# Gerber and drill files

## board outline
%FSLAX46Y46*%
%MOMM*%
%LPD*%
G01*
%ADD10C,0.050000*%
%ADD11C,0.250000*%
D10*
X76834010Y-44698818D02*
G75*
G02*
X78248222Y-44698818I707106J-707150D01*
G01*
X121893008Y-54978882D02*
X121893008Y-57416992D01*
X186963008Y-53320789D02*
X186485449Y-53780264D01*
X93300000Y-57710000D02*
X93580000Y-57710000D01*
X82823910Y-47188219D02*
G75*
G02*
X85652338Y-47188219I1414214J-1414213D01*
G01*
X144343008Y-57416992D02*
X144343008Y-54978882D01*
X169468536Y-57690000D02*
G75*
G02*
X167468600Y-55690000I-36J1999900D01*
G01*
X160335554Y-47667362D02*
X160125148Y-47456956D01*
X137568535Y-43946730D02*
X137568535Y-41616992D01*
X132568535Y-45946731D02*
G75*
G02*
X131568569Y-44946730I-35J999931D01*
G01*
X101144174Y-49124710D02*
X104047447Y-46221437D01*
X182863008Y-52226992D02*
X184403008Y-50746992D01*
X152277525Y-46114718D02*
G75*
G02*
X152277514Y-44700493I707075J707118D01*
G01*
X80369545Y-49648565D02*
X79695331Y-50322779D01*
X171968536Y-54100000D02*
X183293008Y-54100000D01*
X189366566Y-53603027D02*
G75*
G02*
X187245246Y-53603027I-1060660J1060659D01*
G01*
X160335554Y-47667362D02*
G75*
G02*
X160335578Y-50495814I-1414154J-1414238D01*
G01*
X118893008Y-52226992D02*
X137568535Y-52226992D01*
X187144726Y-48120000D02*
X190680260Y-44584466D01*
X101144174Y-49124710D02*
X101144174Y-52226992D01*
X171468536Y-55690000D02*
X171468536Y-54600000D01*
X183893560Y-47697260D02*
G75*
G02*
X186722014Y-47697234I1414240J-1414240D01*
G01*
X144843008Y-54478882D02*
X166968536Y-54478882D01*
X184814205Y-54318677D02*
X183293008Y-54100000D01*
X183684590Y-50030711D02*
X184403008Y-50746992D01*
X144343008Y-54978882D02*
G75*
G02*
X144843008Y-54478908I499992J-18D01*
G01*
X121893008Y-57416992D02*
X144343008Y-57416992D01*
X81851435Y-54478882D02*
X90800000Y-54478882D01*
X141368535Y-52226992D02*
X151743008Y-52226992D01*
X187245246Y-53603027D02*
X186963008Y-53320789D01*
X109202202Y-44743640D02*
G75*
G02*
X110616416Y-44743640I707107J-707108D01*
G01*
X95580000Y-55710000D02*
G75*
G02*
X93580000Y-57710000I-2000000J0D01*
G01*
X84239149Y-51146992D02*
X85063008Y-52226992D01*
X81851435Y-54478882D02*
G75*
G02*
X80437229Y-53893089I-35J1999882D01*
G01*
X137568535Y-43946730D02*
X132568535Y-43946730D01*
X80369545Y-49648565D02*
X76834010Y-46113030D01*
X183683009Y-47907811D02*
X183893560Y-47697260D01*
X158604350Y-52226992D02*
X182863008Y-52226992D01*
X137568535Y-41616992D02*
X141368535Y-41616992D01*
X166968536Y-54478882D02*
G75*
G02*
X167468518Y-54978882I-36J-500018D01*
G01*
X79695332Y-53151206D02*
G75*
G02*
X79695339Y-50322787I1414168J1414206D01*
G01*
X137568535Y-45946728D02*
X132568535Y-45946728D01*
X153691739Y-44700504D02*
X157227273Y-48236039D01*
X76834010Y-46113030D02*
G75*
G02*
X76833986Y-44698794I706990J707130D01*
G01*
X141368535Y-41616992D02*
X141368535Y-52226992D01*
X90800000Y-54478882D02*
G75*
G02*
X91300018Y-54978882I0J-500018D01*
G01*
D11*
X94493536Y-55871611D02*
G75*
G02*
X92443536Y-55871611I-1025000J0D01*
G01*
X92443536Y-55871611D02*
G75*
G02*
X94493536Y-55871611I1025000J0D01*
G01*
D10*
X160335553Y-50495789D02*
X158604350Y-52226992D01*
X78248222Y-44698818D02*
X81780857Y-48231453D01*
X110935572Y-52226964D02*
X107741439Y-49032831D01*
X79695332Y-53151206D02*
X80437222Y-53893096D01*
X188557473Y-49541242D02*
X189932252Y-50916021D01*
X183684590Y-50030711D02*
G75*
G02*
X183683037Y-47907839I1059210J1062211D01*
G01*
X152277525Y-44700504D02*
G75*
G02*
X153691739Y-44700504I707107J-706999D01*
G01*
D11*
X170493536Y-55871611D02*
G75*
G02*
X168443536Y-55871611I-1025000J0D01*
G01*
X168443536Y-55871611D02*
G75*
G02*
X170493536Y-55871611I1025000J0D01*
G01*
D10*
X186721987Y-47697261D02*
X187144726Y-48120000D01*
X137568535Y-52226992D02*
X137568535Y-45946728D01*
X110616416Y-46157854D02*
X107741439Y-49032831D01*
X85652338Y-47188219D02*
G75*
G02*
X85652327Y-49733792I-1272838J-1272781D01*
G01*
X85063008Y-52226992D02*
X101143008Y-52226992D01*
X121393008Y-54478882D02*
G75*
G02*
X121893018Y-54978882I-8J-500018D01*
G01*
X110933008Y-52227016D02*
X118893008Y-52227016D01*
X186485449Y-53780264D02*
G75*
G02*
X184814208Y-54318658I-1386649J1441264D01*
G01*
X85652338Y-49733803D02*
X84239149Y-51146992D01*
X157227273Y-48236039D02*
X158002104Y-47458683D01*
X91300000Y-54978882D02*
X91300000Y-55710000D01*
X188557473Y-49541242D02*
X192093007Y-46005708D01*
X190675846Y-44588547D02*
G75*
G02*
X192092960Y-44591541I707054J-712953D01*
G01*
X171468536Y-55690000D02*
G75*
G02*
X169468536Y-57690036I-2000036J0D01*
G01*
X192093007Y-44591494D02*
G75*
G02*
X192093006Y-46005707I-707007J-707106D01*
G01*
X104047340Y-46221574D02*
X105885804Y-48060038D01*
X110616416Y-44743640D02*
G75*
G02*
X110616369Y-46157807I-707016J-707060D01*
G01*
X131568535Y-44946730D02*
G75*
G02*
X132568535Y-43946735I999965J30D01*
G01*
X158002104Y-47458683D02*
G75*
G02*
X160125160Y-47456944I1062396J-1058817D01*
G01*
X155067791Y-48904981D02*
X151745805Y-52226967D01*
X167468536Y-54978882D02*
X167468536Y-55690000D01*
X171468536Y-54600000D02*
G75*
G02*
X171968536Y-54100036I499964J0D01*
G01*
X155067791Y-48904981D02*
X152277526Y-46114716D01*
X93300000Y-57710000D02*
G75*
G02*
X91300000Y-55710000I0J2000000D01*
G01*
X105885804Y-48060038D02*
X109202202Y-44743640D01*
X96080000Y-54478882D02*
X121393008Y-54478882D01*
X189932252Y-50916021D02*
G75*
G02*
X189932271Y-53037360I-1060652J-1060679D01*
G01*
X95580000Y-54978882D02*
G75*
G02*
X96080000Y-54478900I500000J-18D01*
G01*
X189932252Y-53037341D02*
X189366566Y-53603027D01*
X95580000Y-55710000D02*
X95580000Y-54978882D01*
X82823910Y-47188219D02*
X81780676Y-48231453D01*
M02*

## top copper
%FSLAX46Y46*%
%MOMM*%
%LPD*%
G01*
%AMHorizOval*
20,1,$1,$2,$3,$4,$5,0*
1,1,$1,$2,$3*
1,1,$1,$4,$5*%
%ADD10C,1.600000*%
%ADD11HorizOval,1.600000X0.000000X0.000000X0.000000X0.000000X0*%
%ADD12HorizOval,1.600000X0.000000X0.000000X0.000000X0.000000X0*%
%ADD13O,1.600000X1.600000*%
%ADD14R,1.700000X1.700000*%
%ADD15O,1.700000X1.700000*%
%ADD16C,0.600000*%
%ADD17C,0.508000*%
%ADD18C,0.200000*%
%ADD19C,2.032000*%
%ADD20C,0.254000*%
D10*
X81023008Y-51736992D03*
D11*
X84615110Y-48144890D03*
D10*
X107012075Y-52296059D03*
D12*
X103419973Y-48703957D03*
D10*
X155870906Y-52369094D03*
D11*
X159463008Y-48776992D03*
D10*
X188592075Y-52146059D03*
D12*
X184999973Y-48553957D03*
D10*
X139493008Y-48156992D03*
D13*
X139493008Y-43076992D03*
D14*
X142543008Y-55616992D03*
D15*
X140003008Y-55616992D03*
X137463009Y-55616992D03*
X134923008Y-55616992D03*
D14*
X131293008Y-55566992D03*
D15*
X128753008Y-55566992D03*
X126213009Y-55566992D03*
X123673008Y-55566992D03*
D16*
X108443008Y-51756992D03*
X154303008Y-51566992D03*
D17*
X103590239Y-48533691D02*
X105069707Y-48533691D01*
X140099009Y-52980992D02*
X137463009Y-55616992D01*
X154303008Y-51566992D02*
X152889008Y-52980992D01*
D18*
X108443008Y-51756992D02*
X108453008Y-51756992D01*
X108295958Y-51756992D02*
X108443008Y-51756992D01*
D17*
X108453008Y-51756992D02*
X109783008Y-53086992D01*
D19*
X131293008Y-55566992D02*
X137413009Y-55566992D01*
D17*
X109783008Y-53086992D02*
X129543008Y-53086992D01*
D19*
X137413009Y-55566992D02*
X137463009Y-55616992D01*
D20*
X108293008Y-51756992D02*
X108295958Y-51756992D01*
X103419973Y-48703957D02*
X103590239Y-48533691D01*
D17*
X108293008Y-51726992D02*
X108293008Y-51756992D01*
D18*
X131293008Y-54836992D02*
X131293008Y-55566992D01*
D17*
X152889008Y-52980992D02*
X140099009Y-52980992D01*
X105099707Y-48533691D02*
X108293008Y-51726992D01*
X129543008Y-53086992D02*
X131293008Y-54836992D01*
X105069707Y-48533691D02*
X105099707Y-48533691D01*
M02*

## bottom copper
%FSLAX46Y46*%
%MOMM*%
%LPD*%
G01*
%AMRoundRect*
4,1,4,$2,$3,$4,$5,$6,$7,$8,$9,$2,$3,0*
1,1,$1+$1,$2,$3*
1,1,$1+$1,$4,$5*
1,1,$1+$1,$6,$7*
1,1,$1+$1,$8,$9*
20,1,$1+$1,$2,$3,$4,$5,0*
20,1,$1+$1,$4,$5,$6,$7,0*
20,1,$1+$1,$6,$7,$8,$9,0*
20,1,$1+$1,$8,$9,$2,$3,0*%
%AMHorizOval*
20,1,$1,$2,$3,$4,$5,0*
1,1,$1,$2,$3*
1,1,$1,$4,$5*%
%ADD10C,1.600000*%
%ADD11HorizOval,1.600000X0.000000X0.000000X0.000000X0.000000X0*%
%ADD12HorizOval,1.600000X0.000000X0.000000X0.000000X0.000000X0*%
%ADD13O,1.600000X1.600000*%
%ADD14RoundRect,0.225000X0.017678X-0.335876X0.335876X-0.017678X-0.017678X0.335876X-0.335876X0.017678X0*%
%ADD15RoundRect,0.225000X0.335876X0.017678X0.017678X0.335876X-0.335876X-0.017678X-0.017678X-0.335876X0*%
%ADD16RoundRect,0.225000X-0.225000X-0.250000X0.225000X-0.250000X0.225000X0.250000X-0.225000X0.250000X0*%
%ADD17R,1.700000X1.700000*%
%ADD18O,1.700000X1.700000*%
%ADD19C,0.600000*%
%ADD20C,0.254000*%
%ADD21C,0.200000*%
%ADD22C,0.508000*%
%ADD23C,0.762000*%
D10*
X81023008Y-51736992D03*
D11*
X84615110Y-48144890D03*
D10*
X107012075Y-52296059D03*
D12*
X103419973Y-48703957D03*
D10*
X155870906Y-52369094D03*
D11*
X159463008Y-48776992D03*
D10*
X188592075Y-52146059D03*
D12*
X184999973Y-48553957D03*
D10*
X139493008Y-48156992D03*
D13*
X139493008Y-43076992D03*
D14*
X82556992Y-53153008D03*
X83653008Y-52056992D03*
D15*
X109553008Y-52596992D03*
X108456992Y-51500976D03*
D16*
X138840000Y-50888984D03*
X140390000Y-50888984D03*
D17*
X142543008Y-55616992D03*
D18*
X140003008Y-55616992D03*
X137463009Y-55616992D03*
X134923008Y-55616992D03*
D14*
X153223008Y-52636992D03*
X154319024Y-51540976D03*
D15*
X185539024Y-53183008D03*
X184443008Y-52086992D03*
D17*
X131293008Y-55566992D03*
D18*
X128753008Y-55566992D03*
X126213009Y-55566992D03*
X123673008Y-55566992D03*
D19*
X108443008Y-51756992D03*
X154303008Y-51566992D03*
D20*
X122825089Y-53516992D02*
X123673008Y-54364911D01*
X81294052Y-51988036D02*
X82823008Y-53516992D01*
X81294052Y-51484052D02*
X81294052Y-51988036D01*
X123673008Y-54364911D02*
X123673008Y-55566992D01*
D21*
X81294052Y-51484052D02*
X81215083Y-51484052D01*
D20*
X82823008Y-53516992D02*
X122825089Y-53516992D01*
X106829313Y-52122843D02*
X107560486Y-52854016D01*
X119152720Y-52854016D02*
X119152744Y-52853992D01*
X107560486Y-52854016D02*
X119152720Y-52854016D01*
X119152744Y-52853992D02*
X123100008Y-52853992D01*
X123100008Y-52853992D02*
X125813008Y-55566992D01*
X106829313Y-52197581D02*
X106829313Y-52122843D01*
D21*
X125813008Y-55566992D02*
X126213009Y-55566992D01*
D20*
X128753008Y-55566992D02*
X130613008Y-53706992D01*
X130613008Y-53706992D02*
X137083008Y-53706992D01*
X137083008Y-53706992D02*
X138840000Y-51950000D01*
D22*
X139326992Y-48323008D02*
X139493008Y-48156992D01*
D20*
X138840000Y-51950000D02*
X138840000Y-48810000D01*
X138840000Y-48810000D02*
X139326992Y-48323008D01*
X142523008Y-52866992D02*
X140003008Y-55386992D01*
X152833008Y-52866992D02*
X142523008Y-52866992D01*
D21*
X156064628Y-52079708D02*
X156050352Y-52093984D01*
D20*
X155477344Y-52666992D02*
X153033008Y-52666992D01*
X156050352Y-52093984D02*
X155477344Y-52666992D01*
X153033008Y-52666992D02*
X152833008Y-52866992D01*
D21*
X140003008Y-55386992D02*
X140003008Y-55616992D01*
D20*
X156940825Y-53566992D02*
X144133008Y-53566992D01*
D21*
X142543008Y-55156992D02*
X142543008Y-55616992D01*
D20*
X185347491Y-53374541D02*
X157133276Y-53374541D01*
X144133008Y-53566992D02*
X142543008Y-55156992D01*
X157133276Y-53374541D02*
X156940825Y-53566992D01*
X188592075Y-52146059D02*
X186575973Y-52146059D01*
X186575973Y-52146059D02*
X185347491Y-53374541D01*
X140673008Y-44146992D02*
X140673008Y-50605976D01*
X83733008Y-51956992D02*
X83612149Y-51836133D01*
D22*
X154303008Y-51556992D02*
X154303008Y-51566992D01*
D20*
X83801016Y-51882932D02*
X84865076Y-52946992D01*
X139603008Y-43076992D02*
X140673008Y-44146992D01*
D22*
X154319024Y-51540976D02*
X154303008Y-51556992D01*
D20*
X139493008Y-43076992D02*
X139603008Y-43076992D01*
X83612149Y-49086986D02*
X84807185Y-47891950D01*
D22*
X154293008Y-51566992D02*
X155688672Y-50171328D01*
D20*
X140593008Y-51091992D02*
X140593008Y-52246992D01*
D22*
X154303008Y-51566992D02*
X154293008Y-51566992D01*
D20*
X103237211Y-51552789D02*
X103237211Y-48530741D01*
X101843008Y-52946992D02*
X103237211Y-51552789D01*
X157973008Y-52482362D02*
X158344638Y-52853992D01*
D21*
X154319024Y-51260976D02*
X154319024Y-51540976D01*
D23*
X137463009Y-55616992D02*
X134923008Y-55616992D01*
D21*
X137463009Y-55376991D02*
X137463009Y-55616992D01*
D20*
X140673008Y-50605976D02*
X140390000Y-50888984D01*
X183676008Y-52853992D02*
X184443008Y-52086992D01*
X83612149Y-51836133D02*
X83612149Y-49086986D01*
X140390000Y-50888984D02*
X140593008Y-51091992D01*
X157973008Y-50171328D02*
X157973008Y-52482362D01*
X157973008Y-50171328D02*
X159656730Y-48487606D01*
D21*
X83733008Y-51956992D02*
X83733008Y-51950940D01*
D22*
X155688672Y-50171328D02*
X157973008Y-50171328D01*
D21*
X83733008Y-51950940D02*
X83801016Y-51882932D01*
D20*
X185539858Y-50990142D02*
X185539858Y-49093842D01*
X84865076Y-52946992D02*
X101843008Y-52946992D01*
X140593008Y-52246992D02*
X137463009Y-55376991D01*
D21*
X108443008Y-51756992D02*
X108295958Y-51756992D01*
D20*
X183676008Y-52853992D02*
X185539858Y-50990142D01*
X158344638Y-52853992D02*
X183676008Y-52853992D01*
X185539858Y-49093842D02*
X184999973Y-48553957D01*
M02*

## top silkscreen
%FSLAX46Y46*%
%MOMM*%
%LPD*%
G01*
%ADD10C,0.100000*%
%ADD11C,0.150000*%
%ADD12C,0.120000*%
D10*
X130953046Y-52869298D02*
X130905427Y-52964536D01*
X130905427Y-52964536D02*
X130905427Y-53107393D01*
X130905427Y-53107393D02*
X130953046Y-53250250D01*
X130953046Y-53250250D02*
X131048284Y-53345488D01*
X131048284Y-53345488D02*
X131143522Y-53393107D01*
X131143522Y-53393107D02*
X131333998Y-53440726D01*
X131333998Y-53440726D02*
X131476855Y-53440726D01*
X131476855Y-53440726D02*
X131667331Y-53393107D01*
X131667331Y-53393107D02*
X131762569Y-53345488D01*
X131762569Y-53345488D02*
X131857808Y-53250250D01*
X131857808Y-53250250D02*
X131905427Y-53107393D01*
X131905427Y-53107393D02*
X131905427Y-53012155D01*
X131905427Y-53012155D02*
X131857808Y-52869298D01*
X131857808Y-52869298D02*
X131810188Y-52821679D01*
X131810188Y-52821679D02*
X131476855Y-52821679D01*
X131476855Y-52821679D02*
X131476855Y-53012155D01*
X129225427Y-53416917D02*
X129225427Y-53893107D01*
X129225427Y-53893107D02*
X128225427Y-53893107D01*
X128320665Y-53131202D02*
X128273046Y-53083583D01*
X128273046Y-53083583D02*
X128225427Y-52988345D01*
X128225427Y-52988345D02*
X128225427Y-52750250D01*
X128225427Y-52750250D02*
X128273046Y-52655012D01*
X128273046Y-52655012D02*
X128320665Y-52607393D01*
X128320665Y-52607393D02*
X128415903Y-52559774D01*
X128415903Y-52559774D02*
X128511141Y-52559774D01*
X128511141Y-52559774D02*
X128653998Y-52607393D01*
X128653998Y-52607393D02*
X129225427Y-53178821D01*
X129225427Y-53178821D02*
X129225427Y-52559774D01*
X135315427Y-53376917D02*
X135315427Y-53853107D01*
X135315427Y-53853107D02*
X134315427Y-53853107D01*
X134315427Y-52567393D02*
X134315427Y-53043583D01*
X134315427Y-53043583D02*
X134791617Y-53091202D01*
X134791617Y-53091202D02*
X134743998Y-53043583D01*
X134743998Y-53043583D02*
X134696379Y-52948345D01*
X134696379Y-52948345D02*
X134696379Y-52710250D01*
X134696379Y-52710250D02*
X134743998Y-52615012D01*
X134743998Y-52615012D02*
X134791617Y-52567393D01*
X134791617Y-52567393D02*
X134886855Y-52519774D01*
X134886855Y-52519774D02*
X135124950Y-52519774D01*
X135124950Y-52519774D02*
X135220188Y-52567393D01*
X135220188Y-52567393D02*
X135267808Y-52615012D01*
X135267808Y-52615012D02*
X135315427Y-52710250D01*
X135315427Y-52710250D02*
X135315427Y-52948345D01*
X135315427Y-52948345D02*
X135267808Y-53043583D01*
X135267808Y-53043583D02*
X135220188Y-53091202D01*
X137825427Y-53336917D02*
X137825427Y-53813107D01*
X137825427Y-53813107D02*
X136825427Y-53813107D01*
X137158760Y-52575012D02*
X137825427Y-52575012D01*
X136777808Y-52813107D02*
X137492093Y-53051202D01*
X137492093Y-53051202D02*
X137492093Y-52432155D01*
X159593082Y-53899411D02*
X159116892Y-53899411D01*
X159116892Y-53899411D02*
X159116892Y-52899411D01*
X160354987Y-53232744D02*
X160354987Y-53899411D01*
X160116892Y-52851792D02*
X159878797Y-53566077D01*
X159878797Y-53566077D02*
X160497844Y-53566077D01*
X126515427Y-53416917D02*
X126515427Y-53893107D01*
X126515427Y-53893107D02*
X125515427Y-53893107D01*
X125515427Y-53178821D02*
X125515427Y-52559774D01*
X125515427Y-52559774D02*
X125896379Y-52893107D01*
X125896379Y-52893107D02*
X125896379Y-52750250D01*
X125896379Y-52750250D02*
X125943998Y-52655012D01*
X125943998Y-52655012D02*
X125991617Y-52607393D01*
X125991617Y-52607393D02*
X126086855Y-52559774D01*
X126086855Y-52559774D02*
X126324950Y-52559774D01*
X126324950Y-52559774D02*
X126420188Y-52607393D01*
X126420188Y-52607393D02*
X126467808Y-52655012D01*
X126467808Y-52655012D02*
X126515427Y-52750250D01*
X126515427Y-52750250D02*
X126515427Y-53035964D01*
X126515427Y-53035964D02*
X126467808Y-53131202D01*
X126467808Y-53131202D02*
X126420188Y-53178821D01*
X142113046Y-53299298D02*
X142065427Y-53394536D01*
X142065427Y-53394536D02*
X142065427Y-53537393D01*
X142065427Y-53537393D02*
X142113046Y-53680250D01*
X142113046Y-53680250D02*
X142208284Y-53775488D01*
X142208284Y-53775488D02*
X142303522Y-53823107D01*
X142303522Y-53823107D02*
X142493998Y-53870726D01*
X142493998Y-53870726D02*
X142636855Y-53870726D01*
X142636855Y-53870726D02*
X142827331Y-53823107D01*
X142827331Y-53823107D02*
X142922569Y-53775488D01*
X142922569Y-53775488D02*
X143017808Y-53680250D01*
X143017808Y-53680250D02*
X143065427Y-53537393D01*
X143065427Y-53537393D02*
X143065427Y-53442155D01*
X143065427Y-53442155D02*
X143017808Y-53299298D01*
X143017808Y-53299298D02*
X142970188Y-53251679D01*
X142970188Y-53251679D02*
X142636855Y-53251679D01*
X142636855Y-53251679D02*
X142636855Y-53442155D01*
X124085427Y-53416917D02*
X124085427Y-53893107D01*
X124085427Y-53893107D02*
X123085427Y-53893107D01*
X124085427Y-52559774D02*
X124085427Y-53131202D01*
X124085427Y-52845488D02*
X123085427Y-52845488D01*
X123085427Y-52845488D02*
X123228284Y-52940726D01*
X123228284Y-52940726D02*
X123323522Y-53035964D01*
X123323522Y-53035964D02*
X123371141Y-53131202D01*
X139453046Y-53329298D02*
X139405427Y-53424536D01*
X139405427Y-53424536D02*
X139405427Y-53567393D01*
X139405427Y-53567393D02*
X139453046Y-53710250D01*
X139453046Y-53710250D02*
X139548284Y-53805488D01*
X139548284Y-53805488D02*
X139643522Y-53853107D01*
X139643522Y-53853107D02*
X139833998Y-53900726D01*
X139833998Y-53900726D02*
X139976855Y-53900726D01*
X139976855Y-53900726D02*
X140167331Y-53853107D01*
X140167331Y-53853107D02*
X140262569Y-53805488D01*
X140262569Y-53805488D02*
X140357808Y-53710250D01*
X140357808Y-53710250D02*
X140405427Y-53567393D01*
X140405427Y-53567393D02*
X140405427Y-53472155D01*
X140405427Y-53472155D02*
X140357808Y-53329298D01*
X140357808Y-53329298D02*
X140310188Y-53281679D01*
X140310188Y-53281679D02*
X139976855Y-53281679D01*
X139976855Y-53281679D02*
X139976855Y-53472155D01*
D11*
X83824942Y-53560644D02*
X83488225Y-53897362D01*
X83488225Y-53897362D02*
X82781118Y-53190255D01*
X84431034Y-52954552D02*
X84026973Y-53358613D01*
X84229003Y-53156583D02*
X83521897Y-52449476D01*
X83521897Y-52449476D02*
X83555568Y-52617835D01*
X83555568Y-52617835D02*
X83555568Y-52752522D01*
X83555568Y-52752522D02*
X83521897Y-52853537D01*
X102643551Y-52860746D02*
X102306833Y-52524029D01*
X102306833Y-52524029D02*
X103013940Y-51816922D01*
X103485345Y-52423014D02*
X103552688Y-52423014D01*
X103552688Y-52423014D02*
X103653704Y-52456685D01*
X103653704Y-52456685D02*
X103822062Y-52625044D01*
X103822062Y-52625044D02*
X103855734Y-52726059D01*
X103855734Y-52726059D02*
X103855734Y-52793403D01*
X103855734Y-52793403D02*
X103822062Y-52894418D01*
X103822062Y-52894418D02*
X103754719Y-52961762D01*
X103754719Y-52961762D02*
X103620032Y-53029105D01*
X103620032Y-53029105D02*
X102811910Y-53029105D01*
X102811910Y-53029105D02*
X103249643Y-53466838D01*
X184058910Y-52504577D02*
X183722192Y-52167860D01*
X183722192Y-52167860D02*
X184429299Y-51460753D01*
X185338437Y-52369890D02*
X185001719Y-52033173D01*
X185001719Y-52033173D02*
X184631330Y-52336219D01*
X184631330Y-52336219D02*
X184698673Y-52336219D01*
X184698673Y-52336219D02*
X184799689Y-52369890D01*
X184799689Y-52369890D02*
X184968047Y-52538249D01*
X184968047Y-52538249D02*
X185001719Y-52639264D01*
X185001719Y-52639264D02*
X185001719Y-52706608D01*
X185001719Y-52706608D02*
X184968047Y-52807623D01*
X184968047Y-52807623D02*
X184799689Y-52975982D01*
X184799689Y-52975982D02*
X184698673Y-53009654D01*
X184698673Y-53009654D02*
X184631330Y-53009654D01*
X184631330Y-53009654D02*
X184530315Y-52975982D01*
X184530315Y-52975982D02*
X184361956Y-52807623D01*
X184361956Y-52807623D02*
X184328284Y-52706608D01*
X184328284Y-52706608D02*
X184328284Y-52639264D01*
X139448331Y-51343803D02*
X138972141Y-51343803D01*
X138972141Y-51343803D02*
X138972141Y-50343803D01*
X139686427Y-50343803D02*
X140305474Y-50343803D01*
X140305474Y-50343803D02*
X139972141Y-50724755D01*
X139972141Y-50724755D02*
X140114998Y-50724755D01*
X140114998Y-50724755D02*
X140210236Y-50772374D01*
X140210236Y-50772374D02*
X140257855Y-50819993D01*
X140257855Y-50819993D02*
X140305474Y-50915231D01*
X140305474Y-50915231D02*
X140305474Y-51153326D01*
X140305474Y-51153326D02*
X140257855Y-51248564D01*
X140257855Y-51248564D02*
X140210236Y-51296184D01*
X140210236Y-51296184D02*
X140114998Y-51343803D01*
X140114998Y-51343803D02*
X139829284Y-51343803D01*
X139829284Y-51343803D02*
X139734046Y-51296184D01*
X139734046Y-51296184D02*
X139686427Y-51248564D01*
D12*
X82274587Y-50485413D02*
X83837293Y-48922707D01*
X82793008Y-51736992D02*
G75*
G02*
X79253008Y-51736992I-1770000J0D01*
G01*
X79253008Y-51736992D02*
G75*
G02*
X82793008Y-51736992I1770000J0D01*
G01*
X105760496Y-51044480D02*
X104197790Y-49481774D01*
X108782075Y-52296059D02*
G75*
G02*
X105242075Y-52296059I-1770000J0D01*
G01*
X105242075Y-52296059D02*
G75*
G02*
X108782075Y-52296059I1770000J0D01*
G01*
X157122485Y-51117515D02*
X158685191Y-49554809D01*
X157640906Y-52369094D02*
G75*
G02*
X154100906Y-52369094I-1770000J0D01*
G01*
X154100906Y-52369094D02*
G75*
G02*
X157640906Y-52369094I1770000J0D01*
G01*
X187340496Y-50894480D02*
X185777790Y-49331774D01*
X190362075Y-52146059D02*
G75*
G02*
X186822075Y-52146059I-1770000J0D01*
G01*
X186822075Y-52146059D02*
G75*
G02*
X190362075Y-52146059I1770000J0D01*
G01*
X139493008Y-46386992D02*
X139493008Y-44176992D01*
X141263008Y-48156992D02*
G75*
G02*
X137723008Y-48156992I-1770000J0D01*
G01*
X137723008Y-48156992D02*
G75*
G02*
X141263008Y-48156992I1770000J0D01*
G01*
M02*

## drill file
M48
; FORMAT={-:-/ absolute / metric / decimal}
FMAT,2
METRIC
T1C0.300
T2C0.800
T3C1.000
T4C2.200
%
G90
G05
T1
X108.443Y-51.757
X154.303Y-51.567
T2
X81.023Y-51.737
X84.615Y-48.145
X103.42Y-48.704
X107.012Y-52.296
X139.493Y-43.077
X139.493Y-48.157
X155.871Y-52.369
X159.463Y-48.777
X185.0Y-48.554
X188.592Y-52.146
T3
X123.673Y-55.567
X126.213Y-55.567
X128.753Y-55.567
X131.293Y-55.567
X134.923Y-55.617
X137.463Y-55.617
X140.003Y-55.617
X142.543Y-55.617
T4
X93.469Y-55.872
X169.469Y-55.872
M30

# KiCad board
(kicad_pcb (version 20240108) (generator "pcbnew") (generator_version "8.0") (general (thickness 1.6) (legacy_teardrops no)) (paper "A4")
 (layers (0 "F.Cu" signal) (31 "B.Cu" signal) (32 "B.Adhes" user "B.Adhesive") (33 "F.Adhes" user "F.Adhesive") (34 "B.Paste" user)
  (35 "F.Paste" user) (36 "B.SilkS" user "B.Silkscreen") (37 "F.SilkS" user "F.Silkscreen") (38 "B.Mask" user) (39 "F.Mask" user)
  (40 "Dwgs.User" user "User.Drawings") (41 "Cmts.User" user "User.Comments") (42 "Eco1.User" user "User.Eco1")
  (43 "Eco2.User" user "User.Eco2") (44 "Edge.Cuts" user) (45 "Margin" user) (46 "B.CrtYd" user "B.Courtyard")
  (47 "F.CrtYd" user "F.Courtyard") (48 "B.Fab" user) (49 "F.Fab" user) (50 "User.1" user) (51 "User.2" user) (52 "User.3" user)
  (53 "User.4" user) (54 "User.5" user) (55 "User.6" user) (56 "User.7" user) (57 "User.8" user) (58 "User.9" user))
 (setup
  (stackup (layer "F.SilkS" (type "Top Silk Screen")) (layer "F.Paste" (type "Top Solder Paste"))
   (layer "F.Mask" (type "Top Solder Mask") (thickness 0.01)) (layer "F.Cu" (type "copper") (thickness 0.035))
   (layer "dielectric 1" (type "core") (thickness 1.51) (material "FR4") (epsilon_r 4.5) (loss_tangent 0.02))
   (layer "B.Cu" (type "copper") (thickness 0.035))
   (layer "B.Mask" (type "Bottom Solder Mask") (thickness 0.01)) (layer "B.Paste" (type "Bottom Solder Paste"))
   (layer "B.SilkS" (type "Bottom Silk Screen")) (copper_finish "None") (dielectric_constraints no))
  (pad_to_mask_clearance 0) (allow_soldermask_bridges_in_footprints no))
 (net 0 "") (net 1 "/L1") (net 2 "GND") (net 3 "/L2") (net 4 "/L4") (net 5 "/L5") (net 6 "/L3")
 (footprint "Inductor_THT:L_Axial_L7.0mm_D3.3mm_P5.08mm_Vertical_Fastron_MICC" (layer "F.Cu") (at 81.023008 51.736992 45)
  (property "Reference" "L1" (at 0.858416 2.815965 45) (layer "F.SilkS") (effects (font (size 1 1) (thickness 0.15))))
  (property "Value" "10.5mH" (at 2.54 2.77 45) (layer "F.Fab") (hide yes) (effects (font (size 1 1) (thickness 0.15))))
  (fp_line (start 1.77 0) (end 3.98 0) (stroke (width 0.12) (type solid)) (layer "F.SilkS"))
  (fp_circle (center 0 0) (end 1.77 0) (stroke (width 0.12) (type solid)) (fill none) (layer "F.SilkS"))
  (pad "1" thru_hole circle (at 0 0 45) (size 1.6 1.6) (drill 0.8) (layers "*.Cu" "*.Mask") (remove_unused_layers no) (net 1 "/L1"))
  (pad "2" thru_hole oval (at 5.079999 0 45) (size 1.6 1.6) (drill 0.8) (layers "*.Cu" "*.Mask") (remove_unused_layers no) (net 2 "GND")))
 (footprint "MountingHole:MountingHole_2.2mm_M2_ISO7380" (layer "F.Cu") (at 93.468536 55.871611)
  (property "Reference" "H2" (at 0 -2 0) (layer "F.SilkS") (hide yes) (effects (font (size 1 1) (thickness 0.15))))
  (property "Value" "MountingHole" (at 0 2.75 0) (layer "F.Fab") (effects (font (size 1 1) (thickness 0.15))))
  (pad "" np_thru_hole circle (at 0 0) (size 2.2 2.2) (drill 2.2) (layers "*.Cu" "*.Mask")))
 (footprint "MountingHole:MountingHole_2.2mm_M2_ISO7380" (layer "F.Cu") (at 169.468536 55.871611)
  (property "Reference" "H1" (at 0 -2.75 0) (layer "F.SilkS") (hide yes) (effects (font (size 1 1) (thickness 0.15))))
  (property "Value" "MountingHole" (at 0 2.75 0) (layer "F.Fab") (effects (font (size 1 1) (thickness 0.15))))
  (pad "" np_thru_hole circle (at 0 0) (size 2.2 2.2) (drill 2.2) (layers "*.Cu" "*.Mask")))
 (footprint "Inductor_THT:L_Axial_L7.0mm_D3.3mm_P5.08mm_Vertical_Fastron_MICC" (layer "F.Cu") (at 107.012075 52.296059 135)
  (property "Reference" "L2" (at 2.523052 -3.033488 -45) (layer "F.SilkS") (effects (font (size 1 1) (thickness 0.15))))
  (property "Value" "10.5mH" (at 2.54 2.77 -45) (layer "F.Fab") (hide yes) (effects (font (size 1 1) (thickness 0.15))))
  (fp_line (start 1.77 0) (end 3.98 0) (stroke (width 0.12) (type solid)) (layer "F.SilkS"))
  (fp_circle (center 0 0) (end 1.77 0) (stroke (width 0.12) (type solid)) (fill none) (layer "F.SilkS"))
  (pad "1" thru_hole circle (at 0 0 135) (size 1.6 1.6) (drill 0.8) (layers "*.Cu" "*.Mask") (remove_unused_layers no) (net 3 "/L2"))
  (pad "2" thru_hole oval (at 5.079999 0 135) (size 1.6 1.6) (drill 0.8) (layers "*.Cu" "*.Mask") (remove_unused_layers no) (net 2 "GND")))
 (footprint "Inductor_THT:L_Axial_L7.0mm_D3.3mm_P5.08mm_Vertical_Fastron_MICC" (layer "F.Cu") (at 155.870906 52.369094 45)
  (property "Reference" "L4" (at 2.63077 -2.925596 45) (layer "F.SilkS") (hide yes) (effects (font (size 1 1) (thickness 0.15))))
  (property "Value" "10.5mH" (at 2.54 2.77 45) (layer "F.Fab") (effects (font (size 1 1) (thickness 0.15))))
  (fp_line (start 1.77 0) (end 3.98 0) (stroke (width 0.12) (type solid)) (layer "F.SilkS"))
  (fp_circle (center 0 0) (end 1.77 0) (stroke (width 0.12) (type solid)) (fill none) (layer "F.SilkS"))
  (pad "1" thru_hole circle (at 0 0 45) (size 1.6 1.6) (drill 0.8) (layers "*.Cu" "*.Mask") (remove_unused_layers no) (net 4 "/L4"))
  (pad "2" thru_hole oval (at 5.079999 0 45) (size 1.6 1.6) (drill 0.8) (layers "*.Cu" "*.Mask") (remove_unused_layers no) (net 2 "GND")))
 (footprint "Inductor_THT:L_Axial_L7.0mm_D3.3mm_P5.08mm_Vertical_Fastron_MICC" (layer "F.Cu") (at 188.592075 52.146059 135)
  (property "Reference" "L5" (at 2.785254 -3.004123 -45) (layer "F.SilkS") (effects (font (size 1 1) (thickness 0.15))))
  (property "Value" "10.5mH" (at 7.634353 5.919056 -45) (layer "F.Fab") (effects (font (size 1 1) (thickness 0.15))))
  (fp_line (start 1.77 0) (end 3.98 0) (stroke (width 0.12) (type solid)) (layer "F.SilkS"))
  (fp_circle (center 0 0) (end 1.77 0) (stroke (width 0.12) (type solid)) (fill none) (layer "F.SilkS"))
  (pad "1" thru_hole circle (at 0 0 135) (size 1.6 1.6) (drill 0.8) (layers "*.Cu" "*.Mask") (remove_unused_layers no) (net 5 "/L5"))
  (pad "2" thru_hole oval (at 5.079999 0 135) (size 1.6 1.6) (drill 0.8) (layers "*.Cu" "*.Mask") (remove_unused_layers no) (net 2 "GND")))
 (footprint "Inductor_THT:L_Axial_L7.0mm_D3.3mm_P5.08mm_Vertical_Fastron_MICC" (layer "F.Cu") (at 139.493008 48.156992 90)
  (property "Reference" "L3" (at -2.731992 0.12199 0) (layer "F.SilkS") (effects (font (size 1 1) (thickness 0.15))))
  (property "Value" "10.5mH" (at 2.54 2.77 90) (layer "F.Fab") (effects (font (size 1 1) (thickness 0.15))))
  (fp_line (start 1.77 0) (end 3.98 0) (stroke (width 0.12) (type solid)) (layer "F.SilkS"))
  (fp_circle (center 0 0) (end 1.77 0) (stroke (width 0.12) (type solid)) (fill none) (layer "F.SilkS"))
  (pad "1" thru_hole circle (at 0 0 90) (size 1.6 1.6) (drill 0.8) (layers "*.Cu" "*.Mask") (remove_unused_layers no) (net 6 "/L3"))
  (pad "2" thru_hole oval (at 5.08 0 90) (size 1.6 1.6) (drill 0.8) (layers "*.Cu" "*.Mask") (remove_unused_layers no) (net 2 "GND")))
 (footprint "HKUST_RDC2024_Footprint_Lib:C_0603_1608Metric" (layer "B.Cu") (at 83.105 52.605 45)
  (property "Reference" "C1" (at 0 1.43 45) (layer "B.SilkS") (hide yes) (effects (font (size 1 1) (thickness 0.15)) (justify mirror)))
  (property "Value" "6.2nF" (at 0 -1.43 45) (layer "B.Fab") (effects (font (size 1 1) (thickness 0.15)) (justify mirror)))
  (pad "1" smd roundrect (at -0.775 0 45) (size 0.9 0.95) (layers "B.Cu" "B.Paste" "B.Mask") (roundrect_rratio 0.25) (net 1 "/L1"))
  (pad "2" smd roundrect (at 0.775 0 45) (size 0.9 0.95) (layers "B.Cu" "B.Paste" "B.Mask") (roundrect_rratio 0.25) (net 2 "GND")))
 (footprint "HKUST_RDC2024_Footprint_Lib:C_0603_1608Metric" (layer "B.Cu") (at 109.005 52.048984 135)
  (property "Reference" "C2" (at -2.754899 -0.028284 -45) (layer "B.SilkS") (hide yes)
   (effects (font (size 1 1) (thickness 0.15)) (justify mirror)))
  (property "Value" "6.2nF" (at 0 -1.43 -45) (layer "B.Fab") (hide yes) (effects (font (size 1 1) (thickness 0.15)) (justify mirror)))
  (pad "1" smd roundrect (at -0.775 0 135) (size 0.9 0.95) (layers "B.Cu" "B.Paste" "B.Mask") (roundrect_rratio 0.25) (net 3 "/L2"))
  (pad "2" smd roundrect (at 0.775 0 135) (size 0.9 0.95) (layers "B.Cu" "B.Paste" "B.Mask") (roundrect_rratio 0.25) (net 2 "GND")))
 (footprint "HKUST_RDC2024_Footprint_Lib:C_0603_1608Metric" (layer "B.Cu") (at 139.615 50.888984)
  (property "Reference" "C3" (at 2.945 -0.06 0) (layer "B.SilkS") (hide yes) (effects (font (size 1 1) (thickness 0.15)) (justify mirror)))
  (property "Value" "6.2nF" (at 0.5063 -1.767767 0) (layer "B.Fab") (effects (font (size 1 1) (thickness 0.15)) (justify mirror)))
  (pad "1" smd roundrect (at -0.775 0) (size 0.9 0.95) (layers "B.Cu" "B.Paste" "B.Mask") (roundrect_rratio 0.25) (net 6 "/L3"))
  (pad "2" smd roundrect (at 0.775 0) (size 0.9 0.95) (layers "B.Cu" "B.Paste" "B.Mask") (roundrect_rratio 0.25) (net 2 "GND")))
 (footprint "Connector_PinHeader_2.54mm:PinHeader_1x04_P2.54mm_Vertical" (layer "B.Cu") (at 142.543008 55.616992 90)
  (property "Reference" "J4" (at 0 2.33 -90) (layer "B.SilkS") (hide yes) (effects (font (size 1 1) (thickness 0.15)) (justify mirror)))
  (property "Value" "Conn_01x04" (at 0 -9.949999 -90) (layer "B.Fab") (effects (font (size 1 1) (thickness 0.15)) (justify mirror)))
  (pad "1" thru_hole rect (at 0 0 90) (size 1.7 1.7) (drill 1) (layers "*.Cu" "*.Mask") (remove_unused_layers no) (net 5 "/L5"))
  (pad "2" thru_hole oval (at 0 -2.54 90) (size 1.7 1.7) (drill 1) (layers "*.Cu" "*.Mask") (remove_unused_layers no) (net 4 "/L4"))
  (pad "3" thru_hole oval (at 0 -5.079999 90) (size 1.7 1.7) (drill 1) (layers "*.Cu" "*.Mask") (remove_unused_layers no) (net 2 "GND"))
  (pad "4" thru_hole oval (at 0 -7.62 90) (size 1.7 1.7) (drill 1) (layers "*.Cu" "*.Mask") (remove_unused_layers no) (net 2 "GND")))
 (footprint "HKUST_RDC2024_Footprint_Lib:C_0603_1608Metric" (layer "B.Cu") (at 153.771016 52.088984 45)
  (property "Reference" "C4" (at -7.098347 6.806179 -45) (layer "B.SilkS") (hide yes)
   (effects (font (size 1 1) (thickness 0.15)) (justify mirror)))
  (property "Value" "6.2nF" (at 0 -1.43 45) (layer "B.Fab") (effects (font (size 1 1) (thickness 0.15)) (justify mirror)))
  (pad "1" smd roundrect (at -0.775 0 45) (size 0.9 0.95) (layers "B.Cu" "B.Paste" "B.Mask") (roundrect_rratio 0.25) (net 4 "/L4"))
  (pad "2" smd roundrect (at 0.775 0 45) (size 0.9 0.95) (layers "B.Cu" "B.Paste" "B.Mask") (roundrect_rratio 0.25) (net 2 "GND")))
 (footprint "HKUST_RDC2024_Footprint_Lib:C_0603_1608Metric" (layer "B.Cu") (at 184.991016 52.635 135)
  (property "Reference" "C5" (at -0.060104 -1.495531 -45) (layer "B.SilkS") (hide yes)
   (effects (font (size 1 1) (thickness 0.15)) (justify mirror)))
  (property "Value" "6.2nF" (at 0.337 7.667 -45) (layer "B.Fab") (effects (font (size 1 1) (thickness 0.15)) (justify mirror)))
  (pad "1" smd roundrect (at -0.775 0 135) (size 0.9 0.95) (layers "B.Cu" "B.Paste" "B.Mask") (roundrect_rratio 0.25) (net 5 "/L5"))
  (pad "2" smd roundrect (at 0.775 0 135) (size 0.9 0.95) (layers "B.Cu" "B.Paste" "B.Mask") (roundrect_rratio 0.25) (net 2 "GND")))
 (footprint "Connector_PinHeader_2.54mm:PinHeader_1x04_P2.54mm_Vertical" (layer "B.Cu") (at 131.293008 55.566992 90)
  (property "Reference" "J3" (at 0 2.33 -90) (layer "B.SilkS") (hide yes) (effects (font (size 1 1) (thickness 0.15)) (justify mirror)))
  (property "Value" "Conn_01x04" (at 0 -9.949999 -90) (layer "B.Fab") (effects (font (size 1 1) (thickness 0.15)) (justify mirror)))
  (pad "1" thru_hole rect (at 0 0 90) (size 1.7 1.7) (drill 1) (layers "*.Cu" "*.Mask") (remove_unused_layers no) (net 2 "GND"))
  (pad "2" thru_hole oval (at 0 -2.54 90) (size 1.7 1.7) (drill 1) (layers "*.Cu" "*.Mask") (remove_unused_layers no) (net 6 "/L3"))
  (pad "3" thru_hole oval (at 0 -5.079999 90) (size 1.7 1.7) (drill 1) (layers "*.Cu" "*.Mask") (remove_unused_layers no) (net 3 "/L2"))
  (pad "4" thru_hole oval (at 0 -7.62 90) (size 1.7 1.7) (drill 1) (layers "*.Cu" "*.Mask") (remove_unused_layers no) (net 1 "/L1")))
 (gr_arc (start 76.83401 44.698818) (mid 77.541109 44.405938) (end 78.248222 44.698818) (stroke (width 0.05) (type default))
  (layer "Edge.Cuts"))
 (gr_line (start 121.893008 54.978882) (end 121.893008 57.416992) (stroke (width 0.05) (type default)) (layer "Edge.Cuts"))
 (gr_line (start 186.963008 53.320789) (end 186.485449 53.780264) (stroke (width 0.05) (type default)) (layer "Edge.Cuts"))
 (gr_line (start 93.3 57.71) (end 93.58 57.71) (stroke (width 0.05) (type default)) (layer "Edge.Cuts"))
 (gr_arc (start 82.82391 47.188219) (mid 84.238124 46.602432) (end 85.652338 47.188219) (stroke (width 0.05) (type default))
  (layer "Edge.Cuts"))
 (gr_line (start 144.343008 57.416992) (end 144.343008 54.978882) (stroke (width 0.05) (type default)) (layer "Edge.Cuts"))
 (gr_arc (start 169.468536 57.69) (mid 168.054299 57.104226) (end 167.468536 55.69) (stroke (width 0.05) (type default)) (layer "Edge.Cuts"))
 (gr_line (start 160.335554 47.667362) (end 160.125148 47.456956) (stroke (width 0.05) (type default)) (layer "Edge.Cuts"))
 (gr_line (start 137.568535 43.94673) (end 137.568535 41.616992) (stroke (width 0.05) (type default)) (layer "Edge.Cuts"))
 (gr_arc (start 132.568535 45.946731) (mid 131.861397 45.653849) (end 131.568535 44.94673) (stroke (width 0.05) (type default))
  (layer "Edge.Cuts"))
 (gr_line (start 101.144174 49.12471) (end 104.047447 46.221437) (stroke (width 0.05) (type default)) (layer "Edge.Cuts"))
 (gr_line (start 182.863008 52.226992) (end 184.403008 50.746992) (stroke (width 0.05) (type default)) (layer "Edge.Cuts"))
 (gr_arc (start 152.277525 46.114718) (mid 151.984611 45.407605) (end 152.277525 44.700504) (stroke (width 0.05) (type default))
  (layer "Edge.Cuts"))
 (gr_line (start 80.369545 49.648565) (end 79.695331 50.322779) (stroke (width 0.05) (type default)) (layer "Edge.Cuts"))
 (gr_line (start 171.968536 54.1) (end 183.293008 54.1) (stroke (width 0.05) (type default)) (layer "Edge.Cuts"))
 (gr_arc (start 189.366566 53.603027) (mid 188.305906 54.042367) (end 187.245246 53.603027) (stroke (width 0.05) (type default))
  (layer "Edge.Cuts"))
 (gr_arc (start 160.335554 47.667362) (mid 160.921343 49.081581) (end 160.335553 50.495789) (stroke (width 0.05) (type default))
  (layer "Edge.Cuts"))
 (gr_line (start 118.893008 52.226992) (end 137.568535 52.226992) (stroke (width 0.05) (type default)) (layer "Edge.Cuts"))
 (gr_line (start 187.144726 48.12) (end 190.68026 44.584466) (stroke (width 0.05) (type default)) (layer "Edge.Cuts"))
 (gr_line (start 101.144174 49.12471) (end 101.144174 52.226992) (stroke (width 0.05) (type default)) (layer "Edge.Cuts"))
 (gr_line (start 171.468536 55.69) (end 171.468536 54.6) (stroke (width 0.05) (type default)) (layer "Edge.Cuts"))
 (gr_arc (start 183.89356 47.69726) (mid 185.307774 47.111474) (end 186.721987 47.697261) (stroke (width 0.05) (type default))
  (layer "Edge.Cuts"))
 (gr_line (start 144.843008 54.478882) (end 166.968536 54.478882) (stroke (width 0.05) (type default)) (layer "Edge.Cuts"))
 (gr_line (start 184.814205 54.318677) (end 183.293008 54.1) (stroke (width 0.05) (type default)) (layer "Edge.Cuts"))
 (gr_line (start 183.68459 50.030711) (end 184.403008 50.746992) (stroke (width 0.05) (type default)) (layer "Edge.Cuts"))
 (gr_arc (start 144.343008 54.978882) (mid 144.489455 54.625329) (end 144.843008 54.478882) (stroke (width 0.05) (type default))
  (layer "Edge.Cuts"))
 (gr_line (start 121.893008 57.416992) (end 144.343008 57.416992) (stroke (width 0.05) (type default)) (layer "Edge.Cuts"))
 (gr_line (start 81.851435 54.478882) (end 90.8 54.478882) (stroke (width 0.05) (type default)) (layer "Edge.Cuts"))
 (gr_line (start 141.368535 52.226992) (end 151.743008 52.226992) (stroke (width 0.05) (type default)) (layer "Edge.Cuts"))
 (gr_line (start 187.245246 53.603027) (end 186.963008 53.320789) (stroke (width 0.05) (type default)) (layer "Edge.Cuts"))
 (gr_arc (start 109.202202 44.74364) (mid 109.909309 44.450747) (end 110.616416 44.74364) (stroke (width 0.05) (type default))
  (layer "Edge.Cuts"))
 (gr_arc (start 95.58 55.71) (mid 94.994214 57.124214) (end 93.58 57.71) (stroke (width 0.05) (type default)) (layer "Edge.Cuts"))
 (gr_line (start 84.239149 51.146992) (end 85.063008 52.226992) (stroke (width 0.05) (type default)) (layer "Edge.Cuts"))
 (gr_arc (start 81.851435 54.478882) (mid 81.086062 54.326652) (end 80.437222 53.893096) (stroke (width 0.05) (type default))
  (layer "Edge.Cuts"))
 (gr_line (start 137.568535 43.94673) (end 132.568535 43.94673) (stroke (width 0.05) (type default)) (layer "Edge.Cuts"))
 (gr_line (start 80.369545 49.648565) (end 76.83401 46.11303) (stroke (width 0.05) (type default)) (layer "Edge.Cuts"))
 (gr_line (start 183.683009 47.907811) (end 183.89356 47.69726) (stroke (width 0.05) (type default)) (layer "Edge.Cuts"))
 (gr_line (start 158.60435 52.226992) (end 182.863008 52.226992) (stroke (width 0.05) (type default)) (layer "Edge.Cuts"))
 (gr_line (start 137.568535 41.616992) (end 141.368535 41.616992) (stroke (width 0.05) (type default)) (layer "Edge.Cuts"))
 (gr_arc (start 166.968536 54.478882) (mid 167.322089 54.625329) (end 167.468536 54.978882) (stroke (width 0.05) (type default))
  (layer "Edge.Cuts"))
 (gr_arc (start 79.695332 53.151206) (mid 79.109545 51.736993) (end 79.695331 50.322779) (stroke (width 0.05) (type default))
  (layer "Edge.Cuts"))
 (gr_line (start 137.568535 45.946728) (end 132.568535 45.946728) (stroke (width 0.05) (type default)) (layer "Edge.Cuts"))
 (gr_line (start 153.691739 44.700504) (end 157.227273 48.236039) (stroke (width 0.05) (type default)) (layer "Edge.Cuts"))
 (gr_arc (start 76.83401 46.11303) (mid 76.541095 45.405917) (end 76.83401 44.698818) (stroke (width 0.05) (type default))
  (layer "Edge.Cuts"))
 (gr_line (start 141.368535 41.616992) (end 141.368535 52.226992) (stroke (width 0.05) (type default)) (layer "Edge.Cuts"))
 (gr_arc (start 90.8 54.478882) (mid 91.153553 54.625329) (end 91.3 54.978882) (stroke (width 0.05) (type default)) (layer "Edge.Cuts"))
 (gr_circle (center 93.468536 55.871611) (end 94.493536 55.871611) (stroke (width 0.25) (type default)) (fill none) (layer "Edge.Cuts"))
 (gr_line (start 160.335553 50.495789) (end 158.60435 52.226992) (stroke (width 0.05) (type default)) (layer "Edge.Cuts"))
 (gr_line (start 78.248222 44.698818) (end 81.780857 48.231453) (stroke (width 0.05) (type default)) (layer "Edge.Cuts"))
 (gr_line (start 110.935572 52.226964) (end 107.741439 49.032831) (stroke (width 0.05) (type default)) (layer "Edge.Cuts"))
 (gr_line (start 79.695332 53.151206) (end 80.437222 53.893096) (stroke (width 0.05) (type default)) (layer "Edge.Cuts"))
 (gr_line (start 188.557473 49.541242) (end 189.932252 50.916021) (stroke (width 0.05) (type default)) (layer "Edge.Cuts"))
 (gr_arc (start 183.68459 50.030711) (mid 183.243698 48.969597) (end 183.683009 47.907811) (stroke (width 0.05) (type default))
  (layer "Edge.Cuts"))
 (gr_arc (start 152.277525 44.700504) (mid 152.984632 44.407579) (end 153.691739 44.700504) (stroke (width 0.05) (type default))
  (layer "Edge.Cuts"))
 (gr_circle (center 169.468536 55.871611) (end 170.493536 55.871611) (stroke (width 0.25) (type default)) (fill none) (layer "Edge.Cuts"))
 (gr_line (start 186.721987 47.697261) (end 187.144726 48.12) (stroke (width 0.05) (type default)) (layer "Edge.Cuts"))
 (gr_line (start 137.568535 52.226992) (end 137.568535 45.946728) (stroke (width 0.05) (type default)) (layer "Edge.Cuts"))
 (gr_line (start 110.616416 46.157854) (end 107.741439 49.032831) (stroke (width 0.05) (type default)) (layer "Edge.Cuts"))
 (gr_arc (start 85.652338 47.188219) (mid 86.179546 48.461011) (end 85.652338 49.733803) (stroke (width 0.05) (type default))
  (layer "Edge.Cuts"))
 (gr_line (start 85.063008 52.226992) (end 101.143008 52.226992) (stroke (width 0.05) (type default)) (layer "Edge.Cuts"))
 (gr_arc (start 121.393008 54.478882) (mid 121.746563 54.62533) (end 121.893008 54.978882) (stroke (width 0.05) (type default))
  (layer "Edge.Cuts"))
 (gr_line (start 110.933008 52.227016) (end 118.893008 52.227016) (stroke (width 0.05) (type default)) (layer "Edge.Cuts"))
 (gr_arc (start 186.485449 53.780264) (mid 185.712071 54.242676) (end 184.814205 54.318677) (stroke (width 0.05) (type default))
  (layer "Edge.Cuts"))
 (gr_line (start 85.652338 49.733803) (end 84.239149 51.146992) (stroke (width 0.05) (type default)) (layer "Edge.Cuts"))
 (gr_line (start 157.227273 48.236039) (end 158.002104 47.458683) (stroke (width 0.05) (type default)) (layer "Edge.Cuts"))
 (gr_line (start 91.3 54.978882) (end 91.3 55.71) (stroke (width 0.05) (type default)) (layer "Edge.Cuts"))
 (gr_line (start 188.557473 49.541242) (end 192.093007 46.005708) (stroke (width 0.05) (type default)) (layer "Edge.Cuts"))
 (gr_arc (start 190.675846 44.588547) (mid 191.385035 44.297372) (end 192.093007 44.591494) (stroke (width 0.05) (type default))
  (layer "Edge.Cuts"))
 (gr_arc (start 171.468536 55.69) (mid 170.88275 57.104214) (end 169.468536 57.69) (stroke (width 0.05) (type default)) (layer "Edge.Cuts"))
 (gr_arc (start 192.093007 44.591494) (mid 192.385926 45.298598) (end 192.093007 46.005708) (stroke (width 0.05) (type default))
  (layer "Edge.Cuts"))
 (gr_line (start 104.04734 46.221574) (end 105.885804 48.060038) (stroke (width 0.05) (type default)) (layer "Edge.Cuts"))
 (gr_arc (start 110.616416 44.74364) (mid 110.909341 45.45076) (end 110.616416 46.157854) (stroke (width 0.05) (type default))
  (layer "Edge.Cuts"))
 (gr_arc (start 131.568535 44.94673) (mid 131.861416 44.239608) (end 132.568535 43.94673) (stroke (width 0.05) (type default))
  (layer "Edge.Cuts"))
 (gr_arc (start 158.002104 47.458683) (mid 159.063274 47.017596) (end 160.125148 47.456956) (stroke (width 0.05) (type default))
  (layer "Edge.Cuts"))
 (gr_line (start 155.067791 48.904981) (end 151.745805 52.226967) (stroke (width 0.05) (type default)) (layer "Edge.Cuts"))
 (gr_line (start 167.468536 54.978882) (end 167.468536 55.69) (stroke (width 0.05) (type default)) (layer "Edge.Cuts"))
 (gr_arc (start 171.468536 54.6) (mid 171.614983 54.246447) (end 171.968536 54.1) (stroke (width 0.05) (type default)) (layer "Edge.Cuts"))
 (gr_line (start 155.067791 48.904981) (end 152.277526 46.114716) (stroke (width 0.05) (type default)) (layer "Edge.Cuts"))
 (gr_arc (start 93.3 57.71) (mid 91.885786 57.124214) (end 91.3 55.71) (stroke (width 0.05) (type default)) (layer "Edge.Cuts"))
 (gr_line (start 105.885804 48.060038) (end 109.202202 44.74364) (stroke (width 0.05) (type default)) (layer "Edge.Cuts"))
 (gr_line (start 96.08 54.478882) (end 121.393008 54.478882) (stroke (width 0.05) (type default)) (layer "Edge.Cuts"))
 (gr_arc (start 189.932252 50.916021) (mid 190.371592 51.976681) (end 189.932252 53.037341) (stroke (width 0.05) (type default))
  (layer "Edge.Cuts"))
 (gr_arc (start 95.58 54.978882) (mid 95.726447 54.625329) (end 96.08 54.478882) (stroke (width 0.05) (type default)) (layer "Edge.Cuts"))
 (gr_line (start 189.932252 53.037341) (end 189.366566 53.603027) (stroke (width 0.05) (type default)) (layer "Edge.Cuts"))
 (gr_line (start 95.58 55.71) (end 95.58 54.978882) (stroke (width 0.05) (type default)) (layer "Edge.Cuts"))
 (gr_line (start 82.82391 47.188219) (end 81.780676 48.231453) (stroke (width 0.05) (type default)) (layer "Edge.Cuts"))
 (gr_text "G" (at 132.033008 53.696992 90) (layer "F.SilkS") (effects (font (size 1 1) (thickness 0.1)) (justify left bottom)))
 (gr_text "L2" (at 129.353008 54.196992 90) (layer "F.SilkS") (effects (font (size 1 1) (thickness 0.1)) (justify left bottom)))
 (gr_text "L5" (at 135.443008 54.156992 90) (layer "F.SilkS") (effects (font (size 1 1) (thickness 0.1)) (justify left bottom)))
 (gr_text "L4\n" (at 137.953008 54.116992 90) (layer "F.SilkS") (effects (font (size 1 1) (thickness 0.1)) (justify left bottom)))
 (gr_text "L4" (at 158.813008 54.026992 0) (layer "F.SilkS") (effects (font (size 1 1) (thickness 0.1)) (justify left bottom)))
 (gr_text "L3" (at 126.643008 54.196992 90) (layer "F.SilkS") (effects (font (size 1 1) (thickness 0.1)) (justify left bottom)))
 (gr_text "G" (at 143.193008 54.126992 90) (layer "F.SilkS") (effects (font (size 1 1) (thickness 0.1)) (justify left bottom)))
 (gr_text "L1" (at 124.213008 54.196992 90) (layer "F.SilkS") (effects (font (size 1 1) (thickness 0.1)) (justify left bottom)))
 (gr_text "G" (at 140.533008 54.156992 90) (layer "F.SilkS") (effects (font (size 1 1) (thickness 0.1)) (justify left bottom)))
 (segment (start 122.825089 53.516992) (end 123.673008 54.364911) (width 0.254) (layer "B.Cu") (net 1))
 (segment (start 81.294052 51.988036) (end 82.823008 53.516992) (width 0.254) (layer "B.Cu") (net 1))
 (segment (start 81.294052 51.484052) (end 81.294052 51.988036) (width 0.254) (layer "B.Cu") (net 1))
 (segment (start 123.673008 54.364911) (end 123.673008 55.566992) (width 0.254) (layer "B.Cu") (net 1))
 (segment (start 81.294052 51.484052) (end 81.215083 51.484052) (width 0.2) (layer "B.Cu") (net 1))
 (segment (start 82.823008 53.516992) (end 122.825089 53.516992) (width 0.254) (layer "B.Cu") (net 1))
 (segment (start 106.829313 52.122843) (end 107.560486 52.854016) (width 0.254) (layer "B.Cu") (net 3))
 (segment (start 119.15272 52.854016) (end 119.152744 52.853992) (width 0.254) (layer "B.Cu") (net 3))
 (segment (start 107.560486 52.854016) (end 119.15272 52.854016) (width 0.254) (layer "B.Cu") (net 3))
 (segment (start 119.152744 52.853992) (end 123.100008 52.853992) (width 0.254) (layer "B.Cu") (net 3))
 (segment (start 123.100008 52.853992) (end 125.813008 55.566992) (width 0.254) (layer "B.Cu") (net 3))
 (segment (start 106.829313 52.197581) (end 106.829313 52.122843) (width 0.254) (layer "B.Cu") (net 3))
 (segment (start 125.813008 55.566992) (end 126.213009 55.566992) (width 0.2) (layer "B.Cu") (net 3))
 (segment (start 128.753008 55.566992) (end 130.613008 53.706992) (width 0.254) (layer "B.Cu") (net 6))
 (segment (start 130.613008 53.706992) (end 137.083008 53.706992) (width 0.254) (layer "B.Cu") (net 6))
 (segment (start 137.083008 53.706992) (end 138.84 51.95) (width 0.254) (layer "B.Cu") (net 6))
 (segment (start 139.326992 48.323008) (end 139.493008 48.156992) (width 0.508) (layer "B.Cu") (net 6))
 (segment (start 138.84 51.95) (end 138.84 48.81) (width 0.254) (layer "B.Cu") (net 6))
 (segment (start 138.84 48.81) (end 139.326992 48.323008) (width 0.254) (layer "B.Cu") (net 6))
 (segment (start 142.523008 52.866992) (end 140.003008 55.386992) (width 0.254) (layer "B.Cu") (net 4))
 (segment (start 152.833008 52.866992) (end 142.523008 52.866992) (width 0.254) (layer "B.Cu") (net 4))
 (segment (start 156.064628 52.079708) (end 156.050352 52.093984) (width 0.2) (layer "B.Cu") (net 4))
 (segment (start 155.477344 52.666992) (end 153.033008 52.666992) (width 0.254) (layer "B.Cu") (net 4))
 (segment (start 156.050352 52.093984) (end 155.477344 52.666992) (width 0.254) (layer "B.Cu") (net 4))
 (segment (start 153.033008 52.666992) (end 152.833008 52.866992) (width 0.254) (layer "B.Cu") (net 4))
 (segment (start 140.003008 55.386992) (end 140.003008 55.616992) (width 0.2) (layer "B.Cu") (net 4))
 (segment (start 156.940825 53.566992) (end 144.133008 53.566992) (width 0.254) (layer "B.Cu") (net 5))
 (segment (start 142.543008 55.156992) (end 142.543008 55.616992) (width 0.2) (layer "B.Cu") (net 5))
 (segment (start 185.347491 53.374541) (end 157.133276 53.374541) (width 0.254) (layer "B.Cu") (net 5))
 (segment (start 144.133008 53.566992) (end 142.543008 55.156992) (width 0.254) (layer "B.Cu") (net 5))
 (segment (start 157.133276 53.374541) (end 156.940825 53.566992) (width 0.254) (layer "B.Cu") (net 5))
 (segment (start 188.592075 52.146059) (end 186.575973 52.146059) (width 0.254) (layer "B.Cu") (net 5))
 (segment (start 186.575973 52.146059) (end 185.347491 53.374541) (width 0.254) (layer "B.Cu") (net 5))
 (segment (start 103.590239 48.533691) (end 105.069707 48.533691) (width 0.508) (layer "F.Cu") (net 2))
 (segment (start 140.099009 52.980992) (end 137.463009 55.616992) (width 0.508) (layer "F.Cu") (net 2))
 (segment (start 154.303008 51.566992) (end 152.889008 52.980992) (width 0.508) (layer "F.Cu") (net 2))
 (segment (start 108.443008 51.756992) (end 108.453008 51.756992) (width 0.2) (layer "F.Cu") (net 2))
 (segment (start 108.295958 51.756992) (end 108.443008 51.756992) (width 0.2) (layer "F.Cu") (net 2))
 (segment (start 108.453008 51.756992) (end 109.783008 53.086992) (width 0.508) (layer "F.Cu") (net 2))
 (segment (start 131.293008 55.566992) (end 137.413009 55.566992) (width 2.032) (layer "F.Cu") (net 2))
 (segment (start 109.783008 53.086992) (end 129.543008 53.086992) (width 0.508) (layer "F.Cu") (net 2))
 (segment (start 137.413009 55.566992) (end 137.463009 55.616992) (width 2.032) (layer "F.Cu") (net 2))
 (segment (start 108.293008 51.756992) (end 108.295958 51.756992) (width 0.254) (layer "F.Cu") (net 2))
 (segment (start 103.419973 48.703957) (end 103.590239 48.533691) (width 0.254) (layer "F.Cu") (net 2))
 (segment (start 108.293008 51.726992) (end 108.293008 51.756992) (width 0.508) (layer "F.Cu") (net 2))
 (segment (start 131.293008 54.836992) (end 131.293008 55.566992) (width 0.2) (layer "F.Cu") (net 2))
 (segment (start 152.889008 52.980992) (end 140.099009 52.980992) (width 0.508) (layer "F.Cu") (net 2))
 (segment (start 105.099707 48.533691) (end 108.293008 51.726992) (width 0.508) (layer "F.Cu") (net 2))
 (segment (start 129.543008 53.086992) (end 131.293008 54.836992) (width 0.508) (layer "F.Cu") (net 2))
 (segment (start 105.069707 48.533691) (end 105.099707 48.533691) (width 0.508) (layer "F.Cu") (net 2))
 (via (at 108.443008 51.756992) (size 0.6) (drill 0.3) (layers "F.Cu" "B.Cu") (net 2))
 (via (at 154.303008 51.566992) (size 0.6) (drill 0.3) (layers "F.Cu" "B.Cu") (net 2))
 (segment (start 140.673008 44.146992) (end 140.673008 50.605976) (width 0.254) (layer "B.Cu") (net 2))
 (segment (start 83.733008 51.956992) (end 83.612149 51.836133) (width 0.254) (layer "B.Cu") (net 2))
 (segment (start 154.303008 51.556992) (end 154.303008 51.566992) (width 0.508) (layer "B.Cu") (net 2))
 (segment (start 83.801016 51.882932) (end 84.865076 52.946992) (width 0.254) (layer "B.Cu") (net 2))
 (segment (start 139.603008 43.076992) (end 140.673008 44.146992) (width 0.254) (layer "B.Cu") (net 2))
 (segment (start 154.319024 51.540976) (end 154.303008 51.556992) (width 0.508) (layer "B.Cu") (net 2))
 (segment (start 139.493008 43.076992) (end 139.603008 43.076992) (width 0.254) (layer "B.Cu") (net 2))
 (segment (start 83.612149 49.086986) (end 84.807185 47.89195) (width 0.254) (layer "B.Cu") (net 2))
 (segment (start 154.293008 51.566992) (end 155.688672 50.171328) (width 0.508) (layer "B.Cu") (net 2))
 (segment (start 140.593008 51.091992) (end 140.593008 52.246992) (width 0.254) (layer "B.Cu") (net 2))
 (segment (start 154.303008 51.566992) (end 154.293008 51.566992) (width 0.508) (layer "B.Cu") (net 2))
 (segment (start 103.237211 51.552789) (end 103.237211 48.530741) (width 0.254) (layer "B.Cu") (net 2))
 (segment (start 101.843008 52.946992) (end 103.237211 51.552789) (width 0.254) (layer "B.Cu") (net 2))
 (segment (start 157.973008 52.482362) (end 158.344638 52.853992) (width 0.254) (layer "B.Cu") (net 2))
 (segment (start 154.319024 51.260976) (end 154.319024 51.540976) (width 0.2) (layer "B.Cu") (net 2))
 (segment (start 137.463009 55.616992) (end 134.923008 55.616992) (width 0.762) (layer "B.Cu") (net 2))
 (segment (start 137.463009 55.376991) (end 137.463009 55.616992) (width 0.2) (layer "B.Cu") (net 2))
 (segment (start 140.673008 50.605976) (end 140.39 50.888984) (width 0.254) (layer "B.Cu") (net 2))
 (segment (start 183.676008 52.853992) (end 184.443008 52.086992) (width 0.254) (layer "B.Cu") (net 2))
 (segment (start 83.612149 51.836133) (end 83.612149 49.086986) (width 0.254) (layer "B.Cu") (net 2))
 (segment (start 140.39 50.888984) (end 140.593008 51.091992) (width 0.254) (layer "B.Cu") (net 2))
 (segment (start 157.973008 50.171328) (end 157.973008 52.482362) (width 0.254) (layer "B.Cu") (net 2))
 (segment (start 157.973008 50.171328) (end 159.65673 48.487606) (width 0.254) (layer "B.Cu") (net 2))
 (segment (start 83.733008 51.956992) (end 83.733008 51.95094) (width 0.2) (layer "B.Cu") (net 2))
 (segment (start 155.688672 50.171328) (end 157.973008 50.171328) (width 0.508) (layer "B.Cu") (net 2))
 (segment (start 83.733008 51.95094) (end 83.801016 51.882932) (width 0.2) (layer "B.Cu") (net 2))
 (segment (start 185.539858 50.990142) (end 185.539858 49.093842) (width 0.254) (layer "B.Cu") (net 2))
 (segment (start 84.865076 52.946992) (end 101.843008 52.946992) (width 0.254) (layer "B.Cu") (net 2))
 (segment (start 140.593008 52.246992) (end 137.463009 55.376991) (width 0.254) (layer "B.Cu") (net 2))
 (segment (start 108.443008 51.756992) (end 108.295958 51.756992) (width 0.2) (layer "B.Cu") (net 2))
 (segment (start 183.676008 52.853992) (end 185.539858 50.990142) (width 0.254) (layer "B.Cu") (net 2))
 (segment (start 158.344638 52.853992) (end 183.676008 52.853992) (width 0.254) (layer "B.Cu") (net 2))
 (segment (start 185.539858 49.093842) (end 184.999973 48.553957) (width 0.254) (layer "B.Cu") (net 2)))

